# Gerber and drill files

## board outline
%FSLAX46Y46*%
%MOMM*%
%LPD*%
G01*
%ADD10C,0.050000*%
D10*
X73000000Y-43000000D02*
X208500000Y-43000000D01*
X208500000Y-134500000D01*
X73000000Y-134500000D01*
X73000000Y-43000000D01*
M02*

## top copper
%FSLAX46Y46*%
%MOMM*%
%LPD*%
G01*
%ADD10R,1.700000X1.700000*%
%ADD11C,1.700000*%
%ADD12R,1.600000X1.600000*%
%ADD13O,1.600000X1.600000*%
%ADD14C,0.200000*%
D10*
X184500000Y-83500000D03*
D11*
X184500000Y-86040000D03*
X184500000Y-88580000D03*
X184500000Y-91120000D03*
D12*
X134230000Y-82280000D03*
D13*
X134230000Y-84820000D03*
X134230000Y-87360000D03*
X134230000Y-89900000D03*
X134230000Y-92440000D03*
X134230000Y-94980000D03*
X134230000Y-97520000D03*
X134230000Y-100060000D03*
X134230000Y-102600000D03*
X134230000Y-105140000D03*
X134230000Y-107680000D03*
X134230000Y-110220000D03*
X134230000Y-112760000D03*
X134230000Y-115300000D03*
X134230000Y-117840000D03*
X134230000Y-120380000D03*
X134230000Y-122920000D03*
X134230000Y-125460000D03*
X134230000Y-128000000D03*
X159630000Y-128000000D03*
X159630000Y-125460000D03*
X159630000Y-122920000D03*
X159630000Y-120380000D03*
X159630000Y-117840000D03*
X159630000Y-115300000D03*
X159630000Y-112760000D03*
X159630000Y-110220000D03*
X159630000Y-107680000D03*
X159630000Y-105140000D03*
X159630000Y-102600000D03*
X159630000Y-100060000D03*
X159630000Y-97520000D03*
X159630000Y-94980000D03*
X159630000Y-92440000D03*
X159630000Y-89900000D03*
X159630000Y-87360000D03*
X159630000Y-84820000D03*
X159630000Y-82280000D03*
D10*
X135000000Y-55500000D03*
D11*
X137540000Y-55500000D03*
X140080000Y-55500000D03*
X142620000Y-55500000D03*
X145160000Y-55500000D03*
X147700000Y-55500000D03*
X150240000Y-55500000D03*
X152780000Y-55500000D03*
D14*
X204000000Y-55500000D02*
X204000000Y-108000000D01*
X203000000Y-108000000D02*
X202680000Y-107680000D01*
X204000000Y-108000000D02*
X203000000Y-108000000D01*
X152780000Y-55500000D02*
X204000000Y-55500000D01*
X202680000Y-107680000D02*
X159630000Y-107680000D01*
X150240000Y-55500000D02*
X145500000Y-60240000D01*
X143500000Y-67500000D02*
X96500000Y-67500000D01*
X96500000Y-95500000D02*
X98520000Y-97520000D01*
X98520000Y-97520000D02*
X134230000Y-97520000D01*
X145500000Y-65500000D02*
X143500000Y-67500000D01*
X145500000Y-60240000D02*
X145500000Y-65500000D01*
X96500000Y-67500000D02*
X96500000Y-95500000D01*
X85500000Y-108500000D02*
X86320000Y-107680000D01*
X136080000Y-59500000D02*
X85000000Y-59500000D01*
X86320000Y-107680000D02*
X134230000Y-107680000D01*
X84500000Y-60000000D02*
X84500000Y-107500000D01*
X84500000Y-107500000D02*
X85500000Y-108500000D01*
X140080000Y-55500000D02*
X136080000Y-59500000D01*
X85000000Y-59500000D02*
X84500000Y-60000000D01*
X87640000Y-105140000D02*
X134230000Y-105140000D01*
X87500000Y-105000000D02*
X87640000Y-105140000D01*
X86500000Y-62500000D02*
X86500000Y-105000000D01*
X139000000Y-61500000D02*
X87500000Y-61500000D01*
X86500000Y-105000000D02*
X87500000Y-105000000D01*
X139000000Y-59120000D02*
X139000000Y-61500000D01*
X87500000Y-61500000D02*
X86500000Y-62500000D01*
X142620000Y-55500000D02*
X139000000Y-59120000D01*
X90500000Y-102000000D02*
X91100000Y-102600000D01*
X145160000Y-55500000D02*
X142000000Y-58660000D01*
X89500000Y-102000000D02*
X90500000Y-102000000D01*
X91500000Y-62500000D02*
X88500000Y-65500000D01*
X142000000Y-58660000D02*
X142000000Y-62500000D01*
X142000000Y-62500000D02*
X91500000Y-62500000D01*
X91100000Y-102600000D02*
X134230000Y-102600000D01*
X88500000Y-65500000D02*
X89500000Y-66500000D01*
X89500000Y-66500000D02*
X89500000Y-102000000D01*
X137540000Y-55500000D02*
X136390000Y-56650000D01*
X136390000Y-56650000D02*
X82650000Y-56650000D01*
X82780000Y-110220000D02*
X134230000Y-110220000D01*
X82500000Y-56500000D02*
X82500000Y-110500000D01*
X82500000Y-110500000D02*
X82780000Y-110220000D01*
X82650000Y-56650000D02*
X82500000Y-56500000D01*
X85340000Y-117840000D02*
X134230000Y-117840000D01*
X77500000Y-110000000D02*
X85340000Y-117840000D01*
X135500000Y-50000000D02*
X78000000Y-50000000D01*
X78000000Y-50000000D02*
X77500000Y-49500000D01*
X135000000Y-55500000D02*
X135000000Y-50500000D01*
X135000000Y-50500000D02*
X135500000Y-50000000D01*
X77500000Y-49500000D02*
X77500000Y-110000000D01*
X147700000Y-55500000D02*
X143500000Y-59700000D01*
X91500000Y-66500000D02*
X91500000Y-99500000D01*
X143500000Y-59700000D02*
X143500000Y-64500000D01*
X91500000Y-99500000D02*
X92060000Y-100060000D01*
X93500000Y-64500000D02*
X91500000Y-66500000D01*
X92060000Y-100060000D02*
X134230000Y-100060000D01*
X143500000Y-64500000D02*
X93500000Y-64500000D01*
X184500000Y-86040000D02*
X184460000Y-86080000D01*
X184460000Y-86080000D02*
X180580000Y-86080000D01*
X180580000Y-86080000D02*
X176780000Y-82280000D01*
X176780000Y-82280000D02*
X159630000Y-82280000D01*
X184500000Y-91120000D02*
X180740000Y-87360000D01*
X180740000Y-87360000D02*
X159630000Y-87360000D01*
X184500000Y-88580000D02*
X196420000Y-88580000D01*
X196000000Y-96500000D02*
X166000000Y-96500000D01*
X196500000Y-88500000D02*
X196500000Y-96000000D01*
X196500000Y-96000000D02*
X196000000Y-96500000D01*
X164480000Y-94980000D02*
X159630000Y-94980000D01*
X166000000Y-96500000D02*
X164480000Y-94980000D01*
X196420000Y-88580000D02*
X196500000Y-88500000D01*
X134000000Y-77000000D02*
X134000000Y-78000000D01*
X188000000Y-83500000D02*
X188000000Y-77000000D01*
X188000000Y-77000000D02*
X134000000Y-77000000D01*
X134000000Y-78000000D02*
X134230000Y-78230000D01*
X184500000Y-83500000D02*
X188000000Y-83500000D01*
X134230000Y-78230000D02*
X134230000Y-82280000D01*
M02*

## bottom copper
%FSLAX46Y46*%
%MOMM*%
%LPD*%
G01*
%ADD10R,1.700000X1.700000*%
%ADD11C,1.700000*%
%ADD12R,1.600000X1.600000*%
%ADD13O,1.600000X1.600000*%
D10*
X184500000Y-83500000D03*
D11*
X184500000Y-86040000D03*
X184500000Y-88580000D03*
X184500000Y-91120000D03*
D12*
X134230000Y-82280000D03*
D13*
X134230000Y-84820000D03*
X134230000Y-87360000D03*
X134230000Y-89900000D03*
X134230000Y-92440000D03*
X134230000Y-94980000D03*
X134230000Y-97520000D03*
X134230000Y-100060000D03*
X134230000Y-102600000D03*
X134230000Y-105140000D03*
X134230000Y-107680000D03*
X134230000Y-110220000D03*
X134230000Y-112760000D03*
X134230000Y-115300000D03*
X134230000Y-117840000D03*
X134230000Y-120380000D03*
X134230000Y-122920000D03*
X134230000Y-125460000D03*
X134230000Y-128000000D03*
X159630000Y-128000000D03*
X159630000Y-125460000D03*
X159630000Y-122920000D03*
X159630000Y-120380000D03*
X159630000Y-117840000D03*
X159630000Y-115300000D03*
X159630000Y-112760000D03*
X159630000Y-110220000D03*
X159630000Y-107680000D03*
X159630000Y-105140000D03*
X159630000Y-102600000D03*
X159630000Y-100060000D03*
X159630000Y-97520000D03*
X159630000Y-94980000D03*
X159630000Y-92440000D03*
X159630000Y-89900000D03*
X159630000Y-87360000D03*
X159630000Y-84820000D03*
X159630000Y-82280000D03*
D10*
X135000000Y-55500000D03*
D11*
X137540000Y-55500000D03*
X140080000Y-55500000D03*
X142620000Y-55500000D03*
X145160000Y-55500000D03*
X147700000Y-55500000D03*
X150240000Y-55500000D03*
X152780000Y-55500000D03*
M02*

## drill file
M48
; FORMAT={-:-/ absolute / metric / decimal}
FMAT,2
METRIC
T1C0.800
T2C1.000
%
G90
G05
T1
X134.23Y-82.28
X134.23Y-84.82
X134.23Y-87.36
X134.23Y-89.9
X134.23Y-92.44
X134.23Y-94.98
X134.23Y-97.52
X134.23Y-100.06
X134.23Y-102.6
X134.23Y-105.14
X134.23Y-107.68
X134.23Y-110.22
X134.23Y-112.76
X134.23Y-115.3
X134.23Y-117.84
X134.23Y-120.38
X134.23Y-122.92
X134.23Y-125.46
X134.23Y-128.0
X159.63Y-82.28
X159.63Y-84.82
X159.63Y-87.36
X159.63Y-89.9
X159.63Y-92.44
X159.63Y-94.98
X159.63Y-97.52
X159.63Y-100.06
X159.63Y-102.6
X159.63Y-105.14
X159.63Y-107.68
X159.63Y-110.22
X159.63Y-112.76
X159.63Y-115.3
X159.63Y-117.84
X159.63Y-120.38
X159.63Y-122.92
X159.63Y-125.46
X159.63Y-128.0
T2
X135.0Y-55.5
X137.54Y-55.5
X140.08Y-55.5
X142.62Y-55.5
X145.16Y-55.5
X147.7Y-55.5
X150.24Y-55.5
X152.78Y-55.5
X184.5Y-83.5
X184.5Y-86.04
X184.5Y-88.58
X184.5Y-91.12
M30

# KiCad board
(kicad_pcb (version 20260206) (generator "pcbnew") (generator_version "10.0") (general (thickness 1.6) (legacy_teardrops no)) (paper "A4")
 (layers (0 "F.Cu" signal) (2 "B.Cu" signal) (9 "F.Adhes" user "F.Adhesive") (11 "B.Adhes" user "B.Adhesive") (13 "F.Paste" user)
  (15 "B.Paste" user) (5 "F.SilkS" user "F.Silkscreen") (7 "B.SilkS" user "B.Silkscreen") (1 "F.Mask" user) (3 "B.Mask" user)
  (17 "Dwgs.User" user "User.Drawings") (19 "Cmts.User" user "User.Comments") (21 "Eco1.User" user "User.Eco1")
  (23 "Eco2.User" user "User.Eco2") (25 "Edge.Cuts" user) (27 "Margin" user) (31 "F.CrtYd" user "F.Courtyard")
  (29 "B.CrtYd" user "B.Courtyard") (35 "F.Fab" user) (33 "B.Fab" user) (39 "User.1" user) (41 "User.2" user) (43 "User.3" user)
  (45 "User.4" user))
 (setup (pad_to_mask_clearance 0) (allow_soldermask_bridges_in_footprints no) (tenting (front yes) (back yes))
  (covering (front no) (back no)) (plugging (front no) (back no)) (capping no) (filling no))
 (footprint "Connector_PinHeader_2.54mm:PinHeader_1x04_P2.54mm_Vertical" (layer "F.Cu") (at 184.5 83.5)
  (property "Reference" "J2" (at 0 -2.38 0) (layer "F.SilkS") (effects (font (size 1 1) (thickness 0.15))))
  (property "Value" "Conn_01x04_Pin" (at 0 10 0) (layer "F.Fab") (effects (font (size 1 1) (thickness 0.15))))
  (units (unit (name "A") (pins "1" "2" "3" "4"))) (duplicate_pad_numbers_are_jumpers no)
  (pad "1" thru_hole rect (at 0 0) (size 1.7 1.7) (drill 1) (layers "*.Cu" "*.Mask") (remove_unused_layers no) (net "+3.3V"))
  (pad "2" thru_hole circle (at 0 2.54) (size 1.7 1.7) (drill 1) (layers "*.Cu" "*.Mask") (remove_unused_layers no) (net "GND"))
  (pad "3" thru_hole circle (at 0 5.08) (size 1.7 1.7) (drill 1) (layers "*.Cu" "*.Mask") (remove_unused_layers no) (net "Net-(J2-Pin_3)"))
  (pad "4" thru_hole circle (at 0 7.62) (size 1.7 1.7) (drill 1) (layers "*.Cu" "*.Mask") (remove_unused_layers no) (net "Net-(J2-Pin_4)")))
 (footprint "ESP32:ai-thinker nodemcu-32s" (layer "F.Cu") (at 134.23 82.28)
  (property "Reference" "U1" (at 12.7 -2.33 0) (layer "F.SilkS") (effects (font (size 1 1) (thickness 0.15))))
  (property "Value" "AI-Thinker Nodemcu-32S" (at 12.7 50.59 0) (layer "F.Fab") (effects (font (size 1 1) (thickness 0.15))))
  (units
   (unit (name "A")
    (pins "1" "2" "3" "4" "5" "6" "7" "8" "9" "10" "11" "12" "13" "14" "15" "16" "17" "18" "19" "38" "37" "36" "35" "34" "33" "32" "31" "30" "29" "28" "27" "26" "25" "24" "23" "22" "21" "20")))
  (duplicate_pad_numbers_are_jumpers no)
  (pad "1" thru_hole rect (at 0 0) (size 1.6 1.6) (drill 0.8) (layers "*.Cu" "*.Mask") (remove_unused_layers no) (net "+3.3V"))
  (pad "2" thru_hole oval (at 0 2.54) (size 1.6 1.6) (drill 0.8) (layers "*.Cu" "*.Mask") (remove_unused_layers no)
   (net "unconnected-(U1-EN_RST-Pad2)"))
  (pad "3" thru_hole oval (at 0 5.08) (size 1.6 1.6) (drill 0.8) (layers "*.Cu" "*.Mask") (remove_unused_layers no)
   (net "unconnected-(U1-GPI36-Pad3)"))
  (pad "4" thru_hole oval (at 0 7.62) (size 1.6 1.6) (drill 0.8) (layers "*.Cu" "*.Mask") (remove_unused_layers no)
   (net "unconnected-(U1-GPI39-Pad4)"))
  (pad "5" thru_hole oval (at 0 10.16) (size 1.6 1.6) (drill 0.8) (layers "*.Cu" "*.Mask") (remove_unused_layers no)
   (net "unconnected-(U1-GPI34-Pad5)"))
  (pad "6" thru_hole oval (at 0 12.7) (size 1.6 1.6) (drill 0.8) (layers "*.Cu" "*.Mask") (remove_unused_layers no)
   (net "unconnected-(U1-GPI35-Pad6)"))
  (pad "7" thru_hole oval (at 0 15.24) (size 1.6 1.6) (drill 0.8) (layers "*.Cu" "*.Mask") (remove_unused_layers no) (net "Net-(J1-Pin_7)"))
  (pad "8" thru_hole oval (at 0 17.78) (size 1.6 1.6) (drill 0.8) (layers "*.Cu" "*.Mask") (remove_unused_layers no) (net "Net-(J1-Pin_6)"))
  (pad "9" thru_hole oval (at 0 20.32) (size 1.6 1.6) (drill 0.8) (layers "*.Cu" "*.Mask") (remove_unused_layers no) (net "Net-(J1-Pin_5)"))
  (pad "10" thru_hole oval (at 0 22.86) (size 1.6 1.6) (drill 0.8) (layers "*.Cu" "*.Mask") (remove_unused_layers no) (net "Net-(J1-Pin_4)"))
  (pad "11" thru_hole oval (at 0 25.4) (size 1.6 1.6) (drill 0.8) (layers "*.Cu" "*.Mask") (remove_unused_layers no) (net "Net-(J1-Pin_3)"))
  (pad "12" thru_hole oval (at 0 27.94) (size 1.6 1.6) (drill 0.8) (layers "*.Cu" "*.Mask") (remove_unused_layers no) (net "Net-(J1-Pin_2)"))
  (pad "13" thru_hole oval (at 0 30.48) (size 1.6 1.6) (drill 0.8) (layers "*.Cu" "*.Mask") (remove_unused_layers no)
   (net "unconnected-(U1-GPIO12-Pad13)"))
  (pad "14" thru_hole oval (at 0 33.02) (size 1.6 1.6) (drill 0.8) (layers "*.Cu" "*.Mask") (remove_unused_layers no)
   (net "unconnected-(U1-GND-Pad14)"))
  (pad "15" thru_hole oval (at 0 35.56) (size 1.6 1.6) (drill 0.8) (layers "*.Cu" "*.Mask") (remove_unused_layers no) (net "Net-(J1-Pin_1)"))
  (pad "16" thru_hole oval (at 0 38.1) (size 1.6 1.6) (drill 0.8) (layers "*.Cu" "*.Mask") (remove_unused_layers no)
   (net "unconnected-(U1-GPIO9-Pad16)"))
  (pad "17" thru_hole oval (at 0 40.64) (size 1.6 1.6) (drill 0.8) (layers "*.Cu" "*.Mask") (remove_unused_layers no)
   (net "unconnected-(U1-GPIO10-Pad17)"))
  (pad "18" thru_hole oval (at 0 43.18) (size 1.6 1.6) (drill 0.8) (layers "*.Cu" "*.Mask") (remove_unused_layers no)
   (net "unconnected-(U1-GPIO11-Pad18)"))
  (pad "19" thru_hole oval (at 0 45.72) (size 1.6 1.6) (drill 0.8) (layers "*.Cu" "*.Mask") (remove_unused_layers no)
   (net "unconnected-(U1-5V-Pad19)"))
  (pad "20" thru_hole oval (at 25.4 45.72) (size 1.6 1.6) (drill 0.8) (layers "*.Cu" "*.Mask") (remove_unused_layers no)
   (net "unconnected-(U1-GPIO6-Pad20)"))
  (pad "21" thru_hole oval (at 25.4 43.18) (size 1.6 1.6) (drill 0.8) (layers "*.Cu" "*.Mask") (remove_unused_layers no)
   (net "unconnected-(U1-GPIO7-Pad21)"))
  (pad "22" thru_hole oval (at 25.4 40.64) (size 1.6 1.6) (drill 0.8) (layers "*.Cu" "*.Mask") (remove_unused_layers no)
   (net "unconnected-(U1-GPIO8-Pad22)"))
  (pad "23" thru_hole oval (at 25.4 38.1) (size 1.6 1.6) (drill 0.8) (layers "*.Cu" "*.Mask") (remove_unused_layers no)
   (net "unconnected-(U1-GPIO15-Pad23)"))
  (pad "24" thru_hole oval (at 25.4 35.56) (size 1.6 1.6) (drill 0.8) (layers "*.Cu" "*.Mask") (remove_unused_layers no)
   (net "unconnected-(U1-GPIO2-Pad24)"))
  (pad "25" thru_hole oval (at 25.4 33.02) (size 1.6 1.6) (drill 0.8) (layers "*.Cu" "*.Mask") (remove_unused_layers no)
   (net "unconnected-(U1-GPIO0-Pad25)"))
  (pad "26" thru_hole oval (at 25.4 30.48) (size 1.6 1.6) (drill 0.8) (layers "*.Cu" "*.Mask") (remove_unused_layers no)
   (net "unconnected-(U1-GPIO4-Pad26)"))
  (pad "27" thru_hole oval (at 25.4 27.94) (size 1.6 1.6) (drill 0.8) (layers "*.Cu" "*.Mask") (remove_unused_layers no)
   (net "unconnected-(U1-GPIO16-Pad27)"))
  (pad "28" thru_hole oval (at 25.4 25.4) (size 1.6 1.6) (drill 0.8) (layers "*.Cu" "*.Mask") (remove_unused_layers no)
   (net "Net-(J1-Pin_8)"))
  (pad "29" thru_hole oval (at 25.4 22.86) (size 1.6 1.6) (drill 0.8) (layers "*.Cu" "*.Mask") (remove_unused_layers no)
   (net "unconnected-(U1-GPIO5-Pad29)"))
  (pad "30" thru_hole oval (at 25.4 20.32) (size 1.6 1.6) (drill 0.8) (layers "*.Cu" "*.Mask") (remove_unused_layers no)
   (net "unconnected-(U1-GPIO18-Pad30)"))
  (pad "31" thru_hole oval (at 25.4 17.78) (size 1.6 1.6) (drill 0.8) (layers "*.Cu" "*.Mask") (remove_unused_layers no)
   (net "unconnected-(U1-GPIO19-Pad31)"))
  (pad "32" thru_hole oval (at 25.4 15.24) (size 1.6 1.6) (drill 0.8) (layers "*.Cu" "*.Mask") (remove_unused_layers no)
   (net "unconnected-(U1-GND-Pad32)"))
  (pad "33" thru_hole oval (at 25.4 12.7) (size 1.6 1.6) (drill 0.8) (layers "*.Cu" "*.Mask") (remove_unused_layers no)
   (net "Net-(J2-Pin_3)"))
  (pad "34" thru_hole oval (at 25.4 10.16) (size 1.6 1.6) (drill 0.8) (layers "*.Cu" "*.Mask") (remove_unused_layers no)
   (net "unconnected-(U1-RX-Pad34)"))
  (pad "35" thru_hole oval (at 25.4 7.62) (size 1.6 1.6) (drill 0.8) (layers "*.Cu" "*.Mask") (remove_unused_layers no)
   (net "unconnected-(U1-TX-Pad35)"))
  (pad "36" thru_hole oval (at 25.4 5.08) (size 1.6 1.6) (drill 0.8) (layers "*.Cu" "*.Mask") (remove_unused_layers no)
   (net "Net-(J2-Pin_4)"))
  (pad "37" thru_hole oval (at 25.4 2.54) (size 1.6 1.6) (drill 0.8) (layers "*.Cu" "*.Mask") (remove_unused_layers no)
   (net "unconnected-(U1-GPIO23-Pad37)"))
  (pad "38" thru_hole oval (at 25.4 0) (size 1.6 1.6) (drill 0.8) (layers "*.Cu" "*.Mask") (remove_unused_layers no) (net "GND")))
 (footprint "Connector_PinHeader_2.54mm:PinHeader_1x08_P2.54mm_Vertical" (layer "F.Cu") (at 135 55.5 90)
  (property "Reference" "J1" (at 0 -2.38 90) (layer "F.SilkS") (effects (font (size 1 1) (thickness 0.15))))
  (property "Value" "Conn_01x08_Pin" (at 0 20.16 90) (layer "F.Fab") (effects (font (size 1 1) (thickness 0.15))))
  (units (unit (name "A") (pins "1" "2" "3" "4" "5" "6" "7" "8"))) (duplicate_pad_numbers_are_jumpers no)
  (pad "1" thru_hole rect (at 0 0 90) (size 1.7 1.7) (drill 1) (layers "*.Cu" "*.Mask") (remove_unused_layers no) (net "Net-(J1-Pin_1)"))
  (pad "2" thru_hole circle (at 0 2.54 90) (size 1.7 1.7) (drill 1) (layers "*.Cu" "*.Mask") (remove_unused_layers no)
   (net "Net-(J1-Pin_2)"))
  (pad "3" thru_hole circle (at 0 5.08 90) (size 1.7 1.7) (drill 1) (layers "*.Cu" "*.Mask") (remove_unused_layers no)
   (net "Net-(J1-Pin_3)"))
  (pad "4" thru_hole circle (at 0 7.62 90) (size 1.7 1.7) (drill 1) (layers "*.Cu" "*.Mask") (remove_unused_layers no)
   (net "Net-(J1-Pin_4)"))
  (pad "5" thru_hole circle (at 0 10.16 90) (size 1.7 1.7) (drill 1) (layers "*.Cu" "*.Mask") (remove_unused_layers no)
   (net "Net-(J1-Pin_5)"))
  (pad "6" thru_hole circle (at 0 12.7 90) (size 1.7 1.7) (drill 1) (layers "*.Cu" "*.Mask") (remove_unused_layers no)
   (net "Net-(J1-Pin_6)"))
  (pad "7" thru_hole circle (at 0 15.24 90) (size 1.7 1.7) (drill 1) (layers "*.Cu" "*.Mask") (remove_unused_layers no)
   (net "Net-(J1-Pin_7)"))
  (pad "8" thru_hole circle (at 0 17.78 90) (size 1.7 1.7) (drill 1) (layers "*.Cu" "*.Mask") (remove_unused_layers no)
   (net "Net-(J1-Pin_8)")))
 (gr_rect (start 73 43) (end 208.5 134.5) (stroke (width 0.05) (type default)) (fill no) (layer "Edge.Cuts"))
 (segment (start 204 55.5) (end 204 108) (width 0.2) (layer "F.Cu") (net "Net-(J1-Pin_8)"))
 (segment (start 203 108) (end 202.68 107.68) (width 0.2) (layer "F.Cu") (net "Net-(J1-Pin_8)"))
 (segment (start 204 108) (end 203 108) (width 0.2) (layer "F.Cu") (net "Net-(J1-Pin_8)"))
 (segment (start 152.78 55.5) (end 204 55.5) (width 0.2) (layer "F.Cu") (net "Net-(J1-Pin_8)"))
 (segment (start 202.68 107.68) (end 159.63 107.68) (width 0.2) (layer "F.Cu") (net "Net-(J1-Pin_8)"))
 (segment (start 150.24 55.5) (end 145.5 60.24) (width 0.2) (layer "F.Cu") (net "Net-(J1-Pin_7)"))
 (segment (start 143.5 67.5) (end 96.5 67.5) (width 0.2) (layer "F.Cu") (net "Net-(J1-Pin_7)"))
 (segment (start 96.5 95.5) (end 98.52 97.52) (width 0.2) (layer "F.Cu") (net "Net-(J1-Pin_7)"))
 (segment (start 98.52 97.52) (end 134.23 97.52) (width 0.2) (layer "F.Cu") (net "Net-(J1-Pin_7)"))
 (segment (start 145.5 65.5) (end 143.5 67.5) (width 0.2) (layer "F.Cu") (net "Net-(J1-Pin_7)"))
 (segment (start 145.5 60.24) (end 145.5 65.5) (width 0.2) (layer "F.Cu") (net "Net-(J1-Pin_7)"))
 (segment (start 96.5 67.5) (end 96.5 95.5) (width 0.2) (layer "F.Cu") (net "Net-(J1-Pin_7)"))
 (segment (start 85.5 108.5) (end 86.32 107.68) (width 0.2) (layer "F.Cu") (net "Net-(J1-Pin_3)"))
 (segment (start 136.08 59.5) (end 85 59.5) (width 0.2) (layer "F.Cu") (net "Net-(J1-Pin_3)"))
 (segment (start 86.32 107.68) (end 134.23 107.68) (width 0.2) (layer "F.Cu") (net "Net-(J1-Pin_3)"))
 (segment (start 84.5 60) (end 84.5 107.5) (width 0.2) (layer "F.Cu") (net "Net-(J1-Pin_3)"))
 (segment (start 84.5 107.5) (end 85.5 108.5) (width 0.2) (layer "F.Cu") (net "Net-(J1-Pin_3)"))
 (segment (start 140.08 55.5) (end 136.08 59.5) (width 0.2) (layer "F.Cu") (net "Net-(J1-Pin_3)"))
 (segment (start 85 59.5) (end 84.5 60) (width 0.2) (layer "F.Cu") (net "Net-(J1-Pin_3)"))
 (segment (start 87.64 105.14) (end 134.23 105.14) (width 0.2) (layer "F.Cu") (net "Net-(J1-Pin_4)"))
 (segment (start 87.5 105) (end 87.64 105.14) (width 0.2) (layer "F.Cu") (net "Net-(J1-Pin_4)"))
 (segment (start 86.5 62.5) (end 86.5 105) (width 0.2) (layer "F.Cu") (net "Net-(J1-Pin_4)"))
 (segment (start 139 61.5) (end 87.5 61.5) (width 0.2) (layer "F.Cu") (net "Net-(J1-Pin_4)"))
 (segment (start 86.5 105) (end 87.5 105) (width 0.2) (layer "F.Cu") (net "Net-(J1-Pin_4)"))
 (segment (start 139 59.12) (end 139 61.5) (width 0.2) (layer "F.Cu") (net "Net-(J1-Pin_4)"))
 (segment (start 87.5 61.5) (end 86.5 62.5) (width 0.2) (layer "F.Cu") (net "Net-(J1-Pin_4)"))
 (segment (start 142.62 55.5) (end 139 59.12) (width 0.2) (layer "F.Cu") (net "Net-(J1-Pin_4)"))
 (segment (start 90.5 102) (end 91.1 102.6) (width 0.2) (layer "F.Cu") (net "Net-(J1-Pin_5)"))
 (segment (start 145.16 55.5) (end 142 58.66) (width 0.2) (layer "F.Cu") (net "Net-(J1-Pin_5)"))
 (segment (start 89.5 102) (end 90.5 102) (width 0.2) (layer "F.Cu") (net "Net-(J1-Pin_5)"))
 (segment (start 91.5 62.5) (end 88.5 65.5) (width 0.2) (layer "F.Cu") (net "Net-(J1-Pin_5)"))
 (segment (start 142 58.66) (end 142 62.5) (width 0.2) (layer "F.Cu") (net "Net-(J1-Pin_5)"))
 (segment (start 142 62.5) (end 91.5 62.5) (width 0.2) (layer "F.Cu") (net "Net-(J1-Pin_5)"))
 (segment (start 91.1 102.6) (end 134.23 102.6) (width 0.2) (layer "F.Cu") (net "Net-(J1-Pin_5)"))
 (segment (start 88.5 65.5) (end 89.5 66.5) (width 0.2) (layer "F.Cu") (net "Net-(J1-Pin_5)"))
 (segment (start 89.5 66.5) (end 89.5 102) (width 0.2) (layer "F.Cu") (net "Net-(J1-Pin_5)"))
 (segment (start 137.54 55.5) (end 136.39 56.65) (width 0.2) (layer "F.Cu") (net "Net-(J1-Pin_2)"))
 (segment (start 136.39 56.65) (end 82.65 56.65) (width 0.2) (layer "F.Cu") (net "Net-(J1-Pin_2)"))
 (segment (start 82.78 110.22) (end 134.23 110.22) (width 0.2) (layer "F.Cu") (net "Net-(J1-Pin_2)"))
 (segment (start 82.5 56.5) (end 82.5 110.5) (width 0.2) (layer "F.Cu") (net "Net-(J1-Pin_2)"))
 (segment (start 82.5 110.5) (end 82.78 110.22) (width 0.2) (layer "F.Cu") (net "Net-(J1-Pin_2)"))
 (segment (start 82.65 56.65) (end 82.5 56.5) (width 0.2) (layer "F.Cu") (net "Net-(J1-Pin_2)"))
 (segment (start 85.34 117.84) (end 134.23 117.84) (width 0.2) (layer "F.Cu") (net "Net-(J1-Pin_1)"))
 (segment (start 77.5 110) (end 85.34 117.84) (width 0.2) (layer "F.Cu") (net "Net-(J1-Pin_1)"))
 (segment (start 135.5 50) (end 78 50) (width 0.2) (layer "F.Cu") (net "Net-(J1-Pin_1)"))
 (segment (start 78 50) (end 77.5 49.5) (width 0.2) (layer "F.Cu") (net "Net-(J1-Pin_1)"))
 (segment (start 135 55.5) (end 135 50.5) (width 0.2) (layer "F.Cu") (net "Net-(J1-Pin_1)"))
 (segment (start 135 50.5) (end 135.5 50) (width 0.2) (layer "F.Cu") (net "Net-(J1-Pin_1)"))
 (segment (start 77.5 49.5) (end 77.5 110) (width 0.2) (layer "F.Cu") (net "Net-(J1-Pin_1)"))
 (segment (start 147.7 55.5) (end 143.5 59.7) (width 0.2) (layer "F.Cu") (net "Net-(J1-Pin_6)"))
 (segment (start 91.5 66.5) (end 91.5 99.5) (width 0.2) (layer "F.Cu") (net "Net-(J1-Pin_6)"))
 (segment (start 143.5 59.7) (end 143.5 64.5) (width 0.2) (layer "F.Cu") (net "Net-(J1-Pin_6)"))
 (segment (start 91.5 99.5) (end 92.06 100.06) (width 0.2) (layer "F.Cu") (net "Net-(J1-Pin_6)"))
 (segment (start 93.5 64.5) (end 91.5 66.5) (width 0.2) (layer "F.Cu") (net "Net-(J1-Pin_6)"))
 (segment (start 92.06 100.06) (end 134.23 100.06) (width 0.2) (layer "F.Cu") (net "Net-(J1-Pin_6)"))
 (segment (start 143.5 64.5) (end 93.5 64.5) (width 0.2) (layer "F.Cu") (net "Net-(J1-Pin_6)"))
 (segment (start 184.5 86.04) (end 184.46 86.08) (width 0.2) (layer "F.Cu") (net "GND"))
 (segment (start 184.46 86.08) (end 180.58 86.08) (width 0.2) (layer "F.Cu") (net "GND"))
 (segment (start 180.58 86.08) (end 176.78 82.28) (width 0.2) (layer "F.Cu") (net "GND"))
 (segment (start 176.78 82.28) (end 159.63 82.28) (width 0.2) (layer "F.Cu") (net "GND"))
 (segment (start 184.5 91.12) (end 180.74 87.36) (width 0.2) (layer "F.Cu") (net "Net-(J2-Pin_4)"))
 (segment (start 180.74 87.36) (end 159.63 87.36) (width 0.2) (layer "F.Cu") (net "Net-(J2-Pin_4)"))
 (segment (start 184.5 88.58) (end 196.42 88.58) (width 0.2) (layer "F.Cu") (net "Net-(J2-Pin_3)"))
 (segment (start 196 96.5) (end 166 96.5) (width 0.2) (layer "F.Cu") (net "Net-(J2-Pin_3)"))
 (segment (start 196.5 88.5) (end 196.5 96) (width 0.2) (layer "F.Cu") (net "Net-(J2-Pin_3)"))
 (segment (start 196.5 96) (end 196 96.5) (width 0.2) (layer "F.Cu") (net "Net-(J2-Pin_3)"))
 (segment (start 164.48 94.98) (end 159.63 94.98) (width 0.2) (layer "F.Cu") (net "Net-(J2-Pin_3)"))
 (segment (start 166 96.5) (end 164.48 94.98) (width 0.2) (layer "F.Cu") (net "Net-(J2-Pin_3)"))
 (segment (start 196.42 88.58) (end 196.5 88.5) (width 0.2) (layer "F.Cu") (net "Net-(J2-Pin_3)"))
 (segment (start 134 77) (end 134 78) (width 0.2) (layer "F.Cu") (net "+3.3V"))
 (segment (start 188 83.5) (end 188 77) (width 0.2) (layer "F.Cu") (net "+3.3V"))
 (segment (start 188 77) (end 134 77) (width 0.2) (layer "F.Cu") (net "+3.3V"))
 (segment (start 134 78) (end 134.23 78.23) (width 0.2) (layer "F.Cu") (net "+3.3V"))
 (segment (start 184.5 83.5) (end 188 83.5) (width 0.2) (layer "F.Cu") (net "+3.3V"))
 (segment (start 134.23 78.23) (end 134.23 82.28) (width 0.2) (layer "F.Cu") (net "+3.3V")))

